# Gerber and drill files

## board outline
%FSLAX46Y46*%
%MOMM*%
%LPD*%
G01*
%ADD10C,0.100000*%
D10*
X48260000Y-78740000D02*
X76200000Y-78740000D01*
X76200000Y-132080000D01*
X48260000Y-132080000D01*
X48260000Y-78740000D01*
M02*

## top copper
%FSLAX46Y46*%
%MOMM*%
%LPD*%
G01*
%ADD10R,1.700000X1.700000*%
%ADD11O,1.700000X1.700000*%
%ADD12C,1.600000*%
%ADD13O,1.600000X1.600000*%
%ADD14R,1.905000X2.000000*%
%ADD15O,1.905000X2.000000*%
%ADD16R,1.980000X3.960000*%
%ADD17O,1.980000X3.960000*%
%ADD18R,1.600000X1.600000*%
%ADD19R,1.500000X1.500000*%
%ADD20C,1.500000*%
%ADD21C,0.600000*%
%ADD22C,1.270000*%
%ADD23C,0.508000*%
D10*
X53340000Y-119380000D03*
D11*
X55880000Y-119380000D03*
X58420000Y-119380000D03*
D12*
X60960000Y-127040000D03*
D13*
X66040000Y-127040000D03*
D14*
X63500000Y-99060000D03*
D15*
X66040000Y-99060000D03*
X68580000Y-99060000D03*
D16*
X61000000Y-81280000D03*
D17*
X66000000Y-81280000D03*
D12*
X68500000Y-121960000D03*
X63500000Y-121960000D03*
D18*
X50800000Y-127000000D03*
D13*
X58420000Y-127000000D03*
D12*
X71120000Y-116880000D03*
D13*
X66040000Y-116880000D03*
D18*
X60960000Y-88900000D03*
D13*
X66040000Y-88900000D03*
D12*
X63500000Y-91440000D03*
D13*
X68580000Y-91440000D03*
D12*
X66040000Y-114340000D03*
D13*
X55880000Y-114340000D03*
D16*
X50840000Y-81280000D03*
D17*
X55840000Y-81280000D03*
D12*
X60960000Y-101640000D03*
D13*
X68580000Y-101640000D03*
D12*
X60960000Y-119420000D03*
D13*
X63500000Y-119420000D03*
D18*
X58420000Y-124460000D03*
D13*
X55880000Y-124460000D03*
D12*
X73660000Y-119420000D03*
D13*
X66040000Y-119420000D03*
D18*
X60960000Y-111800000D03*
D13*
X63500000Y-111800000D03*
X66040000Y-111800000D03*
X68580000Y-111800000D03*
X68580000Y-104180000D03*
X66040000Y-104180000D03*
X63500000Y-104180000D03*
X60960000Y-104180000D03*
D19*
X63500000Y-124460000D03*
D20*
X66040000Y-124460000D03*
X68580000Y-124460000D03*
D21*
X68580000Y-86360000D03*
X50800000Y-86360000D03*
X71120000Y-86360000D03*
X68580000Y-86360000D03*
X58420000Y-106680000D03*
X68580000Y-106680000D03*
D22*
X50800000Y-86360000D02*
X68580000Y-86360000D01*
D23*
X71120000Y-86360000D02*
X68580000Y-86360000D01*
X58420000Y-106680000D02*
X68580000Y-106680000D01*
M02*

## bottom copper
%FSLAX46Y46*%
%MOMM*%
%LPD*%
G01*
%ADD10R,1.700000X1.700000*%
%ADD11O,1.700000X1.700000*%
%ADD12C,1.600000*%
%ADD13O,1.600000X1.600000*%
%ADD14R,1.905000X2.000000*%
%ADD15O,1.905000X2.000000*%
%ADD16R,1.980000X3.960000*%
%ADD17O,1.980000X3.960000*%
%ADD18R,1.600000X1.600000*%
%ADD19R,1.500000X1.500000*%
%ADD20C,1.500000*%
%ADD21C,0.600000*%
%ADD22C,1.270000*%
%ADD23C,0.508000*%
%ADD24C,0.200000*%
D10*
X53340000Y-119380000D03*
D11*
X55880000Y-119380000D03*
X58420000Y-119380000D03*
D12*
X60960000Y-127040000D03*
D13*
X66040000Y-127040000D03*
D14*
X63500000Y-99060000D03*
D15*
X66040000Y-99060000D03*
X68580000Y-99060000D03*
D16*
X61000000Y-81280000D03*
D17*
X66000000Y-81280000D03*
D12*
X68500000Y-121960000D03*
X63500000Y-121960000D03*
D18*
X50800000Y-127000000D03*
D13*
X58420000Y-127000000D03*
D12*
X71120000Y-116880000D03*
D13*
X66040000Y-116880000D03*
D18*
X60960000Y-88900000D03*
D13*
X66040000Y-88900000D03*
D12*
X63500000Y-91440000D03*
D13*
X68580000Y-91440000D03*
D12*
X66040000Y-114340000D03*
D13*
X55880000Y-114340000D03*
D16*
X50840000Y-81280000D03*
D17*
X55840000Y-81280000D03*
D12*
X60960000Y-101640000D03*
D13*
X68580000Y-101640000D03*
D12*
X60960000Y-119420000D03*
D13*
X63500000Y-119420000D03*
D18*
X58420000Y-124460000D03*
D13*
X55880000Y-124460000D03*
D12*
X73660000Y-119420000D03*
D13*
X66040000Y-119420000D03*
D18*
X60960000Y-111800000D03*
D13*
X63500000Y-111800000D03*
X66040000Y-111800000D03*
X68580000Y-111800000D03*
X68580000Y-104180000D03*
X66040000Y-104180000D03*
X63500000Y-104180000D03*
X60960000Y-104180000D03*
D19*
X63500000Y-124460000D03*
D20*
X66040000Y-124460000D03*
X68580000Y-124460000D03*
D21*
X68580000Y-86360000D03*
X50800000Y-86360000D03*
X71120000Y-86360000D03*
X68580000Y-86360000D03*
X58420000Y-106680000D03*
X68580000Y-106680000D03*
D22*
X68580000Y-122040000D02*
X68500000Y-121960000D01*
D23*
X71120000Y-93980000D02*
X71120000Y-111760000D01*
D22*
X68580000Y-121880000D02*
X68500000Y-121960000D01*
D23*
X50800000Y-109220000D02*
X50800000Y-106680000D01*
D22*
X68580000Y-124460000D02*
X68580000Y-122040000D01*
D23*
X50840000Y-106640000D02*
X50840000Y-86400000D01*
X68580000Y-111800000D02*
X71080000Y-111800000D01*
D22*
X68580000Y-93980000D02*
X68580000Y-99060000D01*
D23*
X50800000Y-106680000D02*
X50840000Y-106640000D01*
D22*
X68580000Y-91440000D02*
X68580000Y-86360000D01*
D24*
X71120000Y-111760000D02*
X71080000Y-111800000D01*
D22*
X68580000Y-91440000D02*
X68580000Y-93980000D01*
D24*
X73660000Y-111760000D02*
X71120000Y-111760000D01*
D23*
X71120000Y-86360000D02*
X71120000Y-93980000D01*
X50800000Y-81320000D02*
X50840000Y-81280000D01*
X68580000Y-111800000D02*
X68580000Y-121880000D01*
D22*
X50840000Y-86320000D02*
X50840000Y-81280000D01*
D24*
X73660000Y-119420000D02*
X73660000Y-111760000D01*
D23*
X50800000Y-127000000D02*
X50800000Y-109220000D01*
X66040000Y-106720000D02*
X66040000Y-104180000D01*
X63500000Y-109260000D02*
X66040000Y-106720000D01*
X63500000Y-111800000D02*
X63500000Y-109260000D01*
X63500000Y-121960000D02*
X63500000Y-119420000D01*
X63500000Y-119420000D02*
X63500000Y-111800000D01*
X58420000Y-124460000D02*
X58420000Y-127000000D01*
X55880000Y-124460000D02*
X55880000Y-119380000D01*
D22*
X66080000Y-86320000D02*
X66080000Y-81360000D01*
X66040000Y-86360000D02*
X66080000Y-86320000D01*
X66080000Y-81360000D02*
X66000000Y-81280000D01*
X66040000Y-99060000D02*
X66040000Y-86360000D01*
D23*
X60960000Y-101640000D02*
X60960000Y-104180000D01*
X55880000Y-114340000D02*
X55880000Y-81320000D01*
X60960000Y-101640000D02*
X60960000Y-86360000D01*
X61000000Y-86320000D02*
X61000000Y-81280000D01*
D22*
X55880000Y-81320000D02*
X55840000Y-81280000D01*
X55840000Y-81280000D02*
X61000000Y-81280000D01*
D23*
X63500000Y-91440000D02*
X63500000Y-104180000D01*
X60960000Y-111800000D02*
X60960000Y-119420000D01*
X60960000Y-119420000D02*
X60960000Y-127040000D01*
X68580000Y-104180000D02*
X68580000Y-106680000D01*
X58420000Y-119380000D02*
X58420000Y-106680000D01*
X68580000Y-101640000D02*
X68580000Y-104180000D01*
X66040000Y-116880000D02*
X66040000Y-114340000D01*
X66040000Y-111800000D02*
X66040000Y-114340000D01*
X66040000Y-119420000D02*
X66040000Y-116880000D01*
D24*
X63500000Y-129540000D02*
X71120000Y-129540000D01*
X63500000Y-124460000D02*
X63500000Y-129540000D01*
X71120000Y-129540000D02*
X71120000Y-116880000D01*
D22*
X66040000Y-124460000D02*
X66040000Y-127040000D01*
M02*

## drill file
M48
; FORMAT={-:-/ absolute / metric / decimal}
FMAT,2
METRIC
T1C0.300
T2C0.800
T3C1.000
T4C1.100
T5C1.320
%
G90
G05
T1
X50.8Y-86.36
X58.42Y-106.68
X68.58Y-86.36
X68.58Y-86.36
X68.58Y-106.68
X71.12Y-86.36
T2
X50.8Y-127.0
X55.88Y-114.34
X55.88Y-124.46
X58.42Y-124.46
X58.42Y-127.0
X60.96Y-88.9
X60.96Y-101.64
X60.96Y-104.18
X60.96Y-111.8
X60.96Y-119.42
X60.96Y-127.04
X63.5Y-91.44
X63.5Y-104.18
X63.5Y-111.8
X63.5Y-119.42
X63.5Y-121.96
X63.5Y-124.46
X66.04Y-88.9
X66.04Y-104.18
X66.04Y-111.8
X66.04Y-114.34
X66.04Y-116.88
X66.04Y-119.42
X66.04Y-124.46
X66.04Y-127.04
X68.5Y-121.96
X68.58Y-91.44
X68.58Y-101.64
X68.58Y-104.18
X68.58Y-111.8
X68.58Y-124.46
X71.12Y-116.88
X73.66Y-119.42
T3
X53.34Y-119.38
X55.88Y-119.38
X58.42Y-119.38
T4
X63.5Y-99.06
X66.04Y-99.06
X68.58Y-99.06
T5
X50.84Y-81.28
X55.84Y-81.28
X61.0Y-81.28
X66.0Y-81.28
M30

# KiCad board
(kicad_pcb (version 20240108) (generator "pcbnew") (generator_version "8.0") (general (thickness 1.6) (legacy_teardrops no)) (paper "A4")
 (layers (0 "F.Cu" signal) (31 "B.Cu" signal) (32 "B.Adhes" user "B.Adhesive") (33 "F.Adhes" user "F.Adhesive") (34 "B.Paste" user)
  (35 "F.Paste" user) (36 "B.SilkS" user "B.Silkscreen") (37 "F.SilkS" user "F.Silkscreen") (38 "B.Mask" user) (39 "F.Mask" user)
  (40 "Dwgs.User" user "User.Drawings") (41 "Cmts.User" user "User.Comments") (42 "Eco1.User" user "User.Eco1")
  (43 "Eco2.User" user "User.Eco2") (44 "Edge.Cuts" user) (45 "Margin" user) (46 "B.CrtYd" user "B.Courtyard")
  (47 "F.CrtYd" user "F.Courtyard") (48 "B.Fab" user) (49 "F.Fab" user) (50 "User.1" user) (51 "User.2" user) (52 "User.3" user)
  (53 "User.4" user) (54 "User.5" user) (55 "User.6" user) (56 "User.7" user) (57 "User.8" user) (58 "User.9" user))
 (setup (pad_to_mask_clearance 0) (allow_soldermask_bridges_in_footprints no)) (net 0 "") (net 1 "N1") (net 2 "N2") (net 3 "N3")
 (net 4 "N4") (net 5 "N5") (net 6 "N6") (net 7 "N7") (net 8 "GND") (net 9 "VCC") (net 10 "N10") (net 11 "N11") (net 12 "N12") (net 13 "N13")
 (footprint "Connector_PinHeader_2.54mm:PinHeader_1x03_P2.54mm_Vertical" (layer "F.Cu") (at 53.34 119.38 90)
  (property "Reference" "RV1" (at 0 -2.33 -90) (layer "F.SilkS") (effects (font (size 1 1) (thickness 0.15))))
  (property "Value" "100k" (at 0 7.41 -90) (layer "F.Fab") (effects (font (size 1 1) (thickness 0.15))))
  (pad "1" thru_hole rect (at 0 0 90) (size 1.7 1.7) (drill 1) (layers "*.Cu" "*.Mask") (remove_unused_layers no) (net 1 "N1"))
  (pad "2" thru_hole oval (at 0 2.54 90) (size 1.7 1.7) (drill 1) (layers "*.Cu" "*.Mask") (remove_unused_layers no) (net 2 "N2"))
  (pad "3" thru_hole oval (at 0 5.08 90) (size 1.7 1.7) (drill 1) (layers "*.Cu" "*.Mask") (remove_unused_layers no) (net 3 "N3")))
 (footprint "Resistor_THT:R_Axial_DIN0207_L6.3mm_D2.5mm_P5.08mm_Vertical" (layer "F.Cu") (at 60.96 127.04)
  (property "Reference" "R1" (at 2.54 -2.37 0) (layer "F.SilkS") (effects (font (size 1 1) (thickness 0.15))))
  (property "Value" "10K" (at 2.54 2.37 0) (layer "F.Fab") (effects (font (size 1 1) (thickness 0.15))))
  (pad "1" thru_hole circle (at 0 0) (size 1.6 1.6) (drill 0.8) (layers "*.Cu" "*.Mask") (remove_unused_layers no) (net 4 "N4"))
  (pad "2" thru_hole oval (at 5.08 0) (size 1.6 1.6) (drill 0.8) (layers "*.Cu" "*.Mask") (remove_unused_layers no) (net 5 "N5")))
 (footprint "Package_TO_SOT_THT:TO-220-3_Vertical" (layer "F.Cu") (at 63.5 99.06)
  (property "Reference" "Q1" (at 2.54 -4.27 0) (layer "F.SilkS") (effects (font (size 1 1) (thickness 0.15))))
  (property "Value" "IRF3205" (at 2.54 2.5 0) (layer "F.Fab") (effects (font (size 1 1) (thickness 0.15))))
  (pad "1" thru_hole rect (at 0 0) (size 1.905 2) (drill 1.1) (layers "*.Cu" "*.Mask") (remove_unused_layers no) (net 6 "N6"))
  (pad "2" thru_hole oval (at 2.54 0) (size 1.905 2) (drill 1.1) (layers "*.Cu" "*.Mask") (remove_unused_layers no) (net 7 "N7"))
  (pad "3" thru_hole oval (at 5.08 0) (size 1.905 2) (drill 1.1) (layers "*.Cu" "*.Mask") (remove_unused_layers no) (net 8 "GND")))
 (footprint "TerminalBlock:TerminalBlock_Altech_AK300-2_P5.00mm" (layer "F.Cu") (at 61 81.28)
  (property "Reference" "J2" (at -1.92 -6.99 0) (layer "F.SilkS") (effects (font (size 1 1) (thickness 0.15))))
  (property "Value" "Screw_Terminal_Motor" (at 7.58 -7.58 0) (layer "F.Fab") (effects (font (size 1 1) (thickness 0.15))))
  (pad "1" thru_hole rect (at 0 0) (size 1.98 3.96) (drill 1.32) (layers "*.Cu" "*.Mask") (remove_unused_layers no) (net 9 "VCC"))
  (pad "2" thru_hole oval (at 5 0) (size 1.98 3.96) (drill 1.32) (layers "*.Cu" "*.Mask") (remove_unused_layers no) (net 7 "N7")))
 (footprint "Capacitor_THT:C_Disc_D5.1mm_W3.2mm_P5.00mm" (layer "F.Cu") (at 68.5 121.96 180)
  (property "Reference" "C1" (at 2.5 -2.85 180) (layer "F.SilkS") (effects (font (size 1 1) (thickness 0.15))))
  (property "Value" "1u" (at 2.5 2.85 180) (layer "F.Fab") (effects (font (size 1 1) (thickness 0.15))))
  (pad "1" thru_hole circle (at 0 0 180) (size 1.6 1.6) (drill 0.8) (layers "*.Cu" "*.Mask") (remove_unused_layers no) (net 8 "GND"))
  (pad "2" thru_hole circle (at 5 0 180) (size 1.6 1.6) (drill 0.8) (layers "*.Cu" "*.Mask") (remove_unused_layers no) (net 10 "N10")))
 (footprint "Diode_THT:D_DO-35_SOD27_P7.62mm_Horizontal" (layer "F.Cu") (at 50.8 127)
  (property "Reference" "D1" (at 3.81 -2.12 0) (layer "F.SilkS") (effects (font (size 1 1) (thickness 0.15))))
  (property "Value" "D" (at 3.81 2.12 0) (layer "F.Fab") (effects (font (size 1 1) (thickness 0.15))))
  (pad "1" thru_hole rect (at 0 0) (size 1.6 1.6) (drill 0.8) (layers "*.Cu" "*.Mask") (remove_unused_layers no) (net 8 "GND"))
  (pad "2" thru_hole oval (at 7.62 0) (size 1.6 1.6) (drill 0.8) (layers "*.Cu" "*.Mask") (remove_unused_layers no) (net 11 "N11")))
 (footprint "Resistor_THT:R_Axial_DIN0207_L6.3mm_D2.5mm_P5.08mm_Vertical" (layer "F.Cu") (at 71.12 116.88 180)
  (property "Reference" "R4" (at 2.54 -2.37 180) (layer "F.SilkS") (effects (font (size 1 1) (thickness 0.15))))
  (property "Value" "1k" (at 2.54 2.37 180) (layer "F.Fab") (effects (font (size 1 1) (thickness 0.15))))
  (pad "1" thru_hole circle (at 0 0 180) (size 1.6 1.6) (drill 0.8) (layers "*.Cu" "*.Mask") (remove_unused_layers no) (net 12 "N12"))
  (pad "2" thru_hole oval (at 5.08 0 180) (size 1.6 1.6) (drill 0.8) (layers "*.Cu" "*.Mask") (remove_unused_layers no) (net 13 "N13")))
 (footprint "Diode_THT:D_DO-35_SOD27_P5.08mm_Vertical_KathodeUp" (layer "F.Cu") (at 60.96 88.9)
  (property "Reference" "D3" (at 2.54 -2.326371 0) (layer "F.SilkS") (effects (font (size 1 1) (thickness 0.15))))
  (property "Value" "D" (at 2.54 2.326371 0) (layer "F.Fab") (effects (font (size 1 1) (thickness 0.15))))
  (pad "1" thru_hole rect (at 0 0) (size 1.6 1.6) (drill 0.8) (layers "*.Cu" "*.Mask") (remove_unused_layers no) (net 9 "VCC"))
  (pad "2" thru_hole oval (at 5.08 0) (size 1.6 1.6) (drill 0.8) (layers "*.Cu" "*.Mask") (remove_unused_layers no) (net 7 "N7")))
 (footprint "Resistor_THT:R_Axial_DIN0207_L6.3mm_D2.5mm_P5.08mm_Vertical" (layer "F.Cu") (at 63.5 91.44)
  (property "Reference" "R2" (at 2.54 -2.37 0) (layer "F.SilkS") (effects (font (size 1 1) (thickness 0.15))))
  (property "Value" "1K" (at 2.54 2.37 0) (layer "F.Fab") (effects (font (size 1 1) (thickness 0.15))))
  (pad "1" thru_hole circle (at 0 0) (size 1.6 1.6) (drill 0.8) (layers "*.Cu" "*.Mask") (remove_unused_layers no) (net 6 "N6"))
  (pad "2" thru_hole oval (at 5.08 0) (size 1.6 1.6) (drill 0.8) (layers "*.Cu" "*.Mask") (remove_unused_layers no) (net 8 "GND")))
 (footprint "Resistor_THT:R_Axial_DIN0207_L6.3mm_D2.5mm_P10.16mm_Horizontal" (layer "F.Cu") (at 66.04 114.34 180)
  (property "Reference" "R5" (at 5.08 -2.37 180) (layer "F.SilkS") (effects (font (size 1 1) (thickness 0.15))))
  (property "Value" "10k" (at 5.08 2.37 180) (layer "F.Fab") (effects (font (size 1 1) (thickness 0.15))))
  (pad "1" thru_hole circle (at 0 0 180) (size 1.6 1.6) (drill 0.8) (layers "*.Cu" "*.Mask") (remove_unused_layers no) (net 13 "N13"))
  (pad "2" thru_hole oval (at 10.16 0 180) (size 1.6 1.6) (drill 0.8) (layers "*.Cu" "*.Mask") (remove_unused_layers no) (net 9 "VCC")))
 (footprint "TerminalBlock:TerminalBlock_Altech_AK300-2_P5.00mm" (layer "F.Cu") (at 50.84 81.28)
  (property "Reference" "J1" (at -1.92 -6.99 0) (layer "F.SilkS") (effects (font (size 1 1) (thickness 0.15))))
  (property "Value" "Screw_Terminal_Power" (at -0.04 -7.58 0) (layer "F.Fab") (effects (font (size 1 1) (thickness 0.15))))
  (pad "1" thru_hole rect (at 0 0) (size 1.98 3.96) (drill 1.32) (layers "*.Cu" "*.Mask") (remove_unused_layers no) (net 8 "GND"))
  (pad "2" thru_hole oval (at 5 0) (size 1.98 3.96) (drill 1.32) (layers "*.Cu" "*.Mask") (remove_unused_layers no) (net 9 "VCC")))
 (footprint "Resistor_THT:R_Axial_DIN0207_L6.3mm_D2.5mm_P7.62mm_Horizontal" (layer "F.Cu") (at 60.96 101.64)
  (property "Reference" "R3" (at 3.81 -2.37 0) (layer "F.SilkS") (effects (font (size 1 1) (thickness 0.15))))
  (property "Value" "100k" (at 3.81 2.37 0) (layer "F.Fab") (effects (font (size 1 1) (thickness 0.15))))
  (pad "1" thru_hole circle (at 0 0) (size 1.6 1.6) (drill 0.8) (layers "*.Cu" "*.Mask") (remove_unused_layers no) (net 9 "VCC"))
  (pad "2" thru_hole oval (at 7.62 0) (size 1.6 1.6) (drill 0.8) (layers "*.Cu" "*.Mask") (remove_unused_layers no) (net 3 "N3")))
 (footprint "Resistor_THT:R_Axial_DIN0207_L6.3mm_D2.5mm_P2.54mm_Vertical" (layer "F.Cu") (at 60.96 119.42)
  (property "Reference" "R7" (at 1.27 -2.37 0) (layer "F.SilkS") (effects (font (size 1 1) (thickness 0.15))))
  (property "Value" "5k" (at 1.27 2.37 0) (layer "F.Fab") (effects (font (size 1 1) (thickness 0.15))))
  (pad "1" thru_hole circle (at 0 0) (size 1.6 1.6) (drill 0.8) (layers "*.Cu" "*.Mask") (remove_unused_layers no) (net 4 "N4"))
  (pad "2" thru_hole oval (at 2.54 0) (size 1.6 1.6) (drill 0.8) (layers "*.Cu" "*.Mask") (remove_unused_layers no) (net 10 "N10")))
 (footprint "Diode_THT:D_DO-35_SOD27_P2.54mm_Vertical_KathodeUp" (layer "F.Cu") (at 58.42 124.46 180)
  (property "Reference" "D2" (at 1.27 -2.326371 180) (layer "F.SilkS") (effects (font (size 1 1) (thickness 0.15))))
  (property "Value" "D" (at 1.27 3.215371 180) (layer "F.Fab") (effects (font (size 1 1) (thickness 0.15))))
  (pad "1" thru_hole rect (at 0 0 180) (size 1.6 1.6) (drill 0.8) (layers "*.Cu" "*.Mask") (remove_unused_layers no) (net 11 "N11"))
  (pad "2" thru_hole oval (at 2.54 0 180) (size 1.6 1.6) (drill 0.8) (layers "*.Cu" "*.Mask") (remove_unused_layers no) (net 2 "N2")))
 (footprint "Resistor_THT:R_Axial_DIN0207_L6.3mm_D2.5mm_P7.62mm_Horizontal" (layer "F.Cu") (at 73.66 119.42 180)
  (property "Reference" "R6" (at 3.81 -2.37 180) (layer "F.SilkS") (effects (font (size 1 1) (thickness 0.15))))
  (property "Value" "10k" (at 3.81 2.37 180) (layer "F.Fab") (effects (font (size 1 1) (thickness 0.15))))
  (pad "1" thru_hole circle (at 0 0 180) (size 1.6 1.6) (drill 0.8) (layers "*.Cu" "*.Mask") (remove_unused_layers no) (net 8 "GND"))
  (pad "2" thru_hole oval (at 7.62 0 180) (size 1.6 1.6) (drill 0.8) (layers "*.Cu" "*.Mask") (remove_unused_layers no) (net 13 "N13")))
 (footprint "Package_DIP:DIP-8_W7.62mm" (layer "F.Cu") (at 60.96 111.8 90)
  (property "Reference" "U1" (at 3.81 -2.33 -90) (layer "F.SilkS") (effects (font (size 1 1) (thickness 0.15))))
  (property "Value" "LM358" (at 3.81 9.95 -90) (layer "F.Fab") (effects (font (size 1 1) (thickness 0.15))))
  (pad "1" thru_hole rect (at 0 0 90) (size 1.6 1.6) (drill 0.8) (layers "*.Cu" "*.Mask") (remove_unused_layers no) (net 4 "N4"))
  (pad "2" thru_hole oval (at 0 2.54 90) (size 1.6 1.6) (drill 0.8) (layers "*.Cu" "*.Mask") (remove_unused_layers no) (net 10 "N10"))
  (pad "3" thru_hole oval (at 0 5.08 90) (size 1.6 1.6) (drill 0.8) (layers "*.Cu" "*.Mask") (remove_unused_layers no) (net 13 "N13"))
  (pad "4" thru_hole oval (at 0 7.62 90) (size 1.6 1.6) (drill 0.8) (layers "*.Cu" "*.Mask") (remove_unused_layers no) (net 8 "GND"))
  (pad "5" thru_hole oval (at 7.62 7.62 90) (size 1.6 1.6) (drill 0.8) (layers "*.Cu" "*.Mask") (remove_unused_layers no) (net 3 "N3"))
  (pad "6" thru_hole oval (at 7.62 5.08 90) (size 1.6 1.6) (drill 0.8) (layers "*.Cu" "*.Mask") (remove_unused_layers no) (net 10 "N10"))
  (pad "7" thru_hole oval (at 7.62 2.54 90) (size 1.6 1.6) (drill 0.8) (layers "*.Cu" "*.Mask") (remove_unused_layers no) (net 6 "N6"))
  (pad "8" thru_hole oval (at 7.62 0 90) (size 1.6 1.6) (drill 0.8) (layers "*.Cu" "*.Mask") (remove_unused_layers no) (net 9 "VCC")))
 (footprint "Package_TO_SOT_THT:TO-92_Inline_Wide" (layer "F.Cu") (at 63.5 124.46)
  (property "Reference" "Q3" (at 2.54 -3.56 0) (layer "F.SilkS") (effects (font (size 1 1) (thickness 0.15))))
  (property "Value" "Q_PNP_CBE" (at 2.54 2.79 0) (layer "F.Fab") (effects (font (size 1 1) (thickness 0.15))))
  (pad "1" thru_hole rect (at 0 0) (size 1.5 1.5) (drill 0.8) (layers "*.Cu" "*.Mask") (remove_unused_layers no) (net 12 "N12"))
  (pad "2" thru_hole circle (at 2.54 0) (size 1.5 1.5) (drill 0.8) (layers "*.Cu" "*.Mask") (remove_unused_layers no) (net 5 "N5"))
  (pad "3" thru_hole circle (at 5.08 0) (size 1.5 1.5) (drill 0.8) (layers "*.Cu" "*.Mask") (remove_unused_layers no) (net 8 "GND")))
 (gr_rect (start 48.26 78.74) (end 76.2 132.08) (stroke (width 0.1) (type default)) (fill none) (layer "Edge.Cuts"))
 (segment (start 50.8 86.36) (end 68.58 86.36) (width 1.27) (layer "F.Cu") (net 8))
 (segment (start 71.12 86.36) (end 68.58 86.36) (width 0.508) (layer "F.Cu") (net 8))
 (via (at 68.58 86.36) (size 0.6) (drill 0.3) (layers "F.Cu" "B.Cu") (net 8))
 (via (at 50.8 86.36) (size 0.6) (drill 0.3) (layers "F.Cu" "B.Cu") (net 8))
 (via (at 71.12 86.36) (size 0.6) (drill 0.3) (layers "F.Cu" "B.Cu") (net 8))
 (via (at 68.58 86.36) (size 0.6) (drill 0.3) (layers "F.Cu" "B.Cu") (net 8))
 (segment (start 68.58 122.04) (end 68.5 121.96) (width 1.27) (layer "B.Cu") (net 8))
 (segment (start 71.12 93.98) (end 71.12 111.76) (width 0.508) (layer "B.Cu") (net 8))
 (segment (start 68.58 121.88) (end 68.5 121.96) (width 1.27) (layer "B.Cu") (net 8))
 (segment (start 50.8 109.22) (end 50.8 106.68) (width 0.508) (layer "B.Cu") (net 8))
 (segment (start 68.58 124.46) (end 68.58 122.04) (width 1.27) (layer "B.Cu") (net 8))
 (segment (start 50.84 106.64) (end 50.84 86.4) (width 0.508) (layer "B.Cu") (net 8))
 (segment (start 68.58 111.8) (end 71.08 111.8) (width 0.508) (layer "B.Cu") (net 8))
 (segment (start 68.58 93.98) (end 68.58 99.06) (width 1.27) (layer "B.Cu") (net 8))
 (segment (start 50.8 106.68) (end 50.84 106.64) (width 0.508) (layer "B.Cu") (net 8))
 (segment (start 68.58 91.44) (end 68.58 86.36) (width 1.27) (layer "B.Cu") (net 8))
 (segment (start 71.12 111.76) (end 71.08 111.8) (width 0.2) (layer "B.Cu") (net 8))
 (segment (start 68.58 91.44) (end 68.58 93.98) (width 1.27) (layer "B.Cu") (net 8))
 (segment (start 73.66 111.76) (end 71.12 111.76) (width 0.2) (layer "B.Cu") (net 8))
 (segment (start 71.12 86.36) (end 71.12 93.98) (width 0.508) (layer "B.Cu") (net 8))
 (segment (start 50.8 81.32) (end 50.84 81.28) (width 0.508) (layer "B.Cu") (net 8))
 (segment (start 68.58 111.8) (end 68.58 121.88) (width 0.508) (layer "B.Cu") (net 8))
 (segment (start 50.84 86.32) (end 50.84 81.28) (width 1.27) (layer "B.Cu") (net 8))
 (segment (start 73.66 119.42) (end 73.66 111.76) (width 0.2) (layer "B.Cu") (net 8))
 (segment (start 50.8 127) (end 50.8 109.22) (width 0.508) (layer "B.Cu") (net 8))
 (segment (start 66.04 106.72) (end 66.04 104.18) (width 0.508) (layer "B.Cu") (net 10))
 (segment (start 63.5 109.26) (end 66.04 106.72) (width 0.508) (layer "B.Cu") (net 10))
 (segment (start 63.5 111.8) (end 63.5 109.26) (width 0.508) (layer "B.Cu") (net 10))
 (segment (start 63.5 121.96) (end 63.5 119.42) (width 0.508) (layer "B.Cu") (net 10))
 (segment (start 63.5 119.42) (end 63.5 111.8) (width 0.508) (layer "B.Cu") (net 10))
 (segment (start 58.42 124.46) (end 58.42 127) (width 0.508) (layer "B.Cu") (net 11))
 (segment (start 55.88 124.46) (end 55.88 119.38) (width 0.508) (layer "B.Cu") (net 2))
 (segment (start 66.08 86.32) (end 66.08 81.36) (width 1.27) (layer "B.Cu") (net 7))
 (segment (start 66.04 86.36) (end 66.08 86.32) (width 1.27) (layer "B.Cu") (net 7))
 (segment (start 66.08 81.36) (end 66 81.28) (width 1.27) (layer "B.Cu") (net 7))
 (segment (start 66.04 99.06) (end 66.04 86.36) (width 1.27) (layer "B.Cu") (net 7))
 (segment (start 60.96 101.64) (end 60.96 104.18) (width 0.508) (layer "B.Cu") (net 9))
 (segment (start 55.88 114.34) (end 55.88 81.32) (width 0.508) (layer "B.Cu") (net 9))
 (segment (start 60.96 101.64) (end 60.96 86.36) (width 0.508) (layer "B.Cu") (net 9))
 (segment (start 61 86.32) (end 61 81.28) (width 0.508) (layer "B.Cu") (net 9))
 (segment (start 55.88 81.32) (end 55.84 81.28) (width 1.27) (layer "B.Cu") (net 9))
 (segment (start 55.84 81.28) (end 61 81.28) (width 1.27) (layer "B.Cu") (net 9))
 (segment (start 63.5 91.44) (end 63.5 104.18) (width 0.508) (layer "B.Cu") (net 6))
 (segment (start 60.96 111.8) (end 60.96 119.42) (width 0.508) (layer "B.Cu") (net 4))
 (segment (start 60.96 119.42) (end 60.96 127.04) (width 0.508) (layer "B.Cu") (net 4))
 (segment (start 58.42 106.68) (end 68.58 106.68) (width 0.508) (layer "F.Cu") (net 3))
 (via (at 58.42 106.68) (size 0.6) (drill 0.3) (layers "F.Cu" "B.Cu") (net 3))
 (via (at 68.58 106.68) (size 0.6) (drill 0.3) (layers "F.Cu" "B.Cu") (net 3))
 (segment (start 68.58 104.18) (end 68.58 106.68) (width 0.508) (layer "B.Cu") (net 3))
 (segment (start 58.42 119.38) (end 58.42 106.68) (width 0.508) (layer "B.Cu") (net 3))
 (segment (start 68.58 101.64) (end 68.58 104.18) (width 0.508) (layer "B.Cu") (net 3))
 (segment (start 66.04 116.88) (end 66.04 114.34) (width 0.508) (layer "B.Cu") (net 13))
 (segment (start 66.04 111.8) (end 66.04 114.34) (width 0.508) (layer "B.Cu") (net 13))
 (segment (start 66.04 119.42) (end 66.04 116.88) (width 0.508) (layer "B.Cu") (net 13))
 (segment (start 63.5 129.54) (end 71.12 129.54) (width 0.2) (layer "B.Cu") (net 12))
 (segment (start 63.5 124.46) (end 63.5 129.54) (width 0.2) (layer "B.Cu") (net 12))
 (segment (start 71.12 129.54) (end 71.12 116.88) (width 0.2) (layer "B.Cu") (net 12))
 (segment (start 66.04 124.46) (end 66.04 127.04) (width 1.27) (layer "B.Cu") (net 5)))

